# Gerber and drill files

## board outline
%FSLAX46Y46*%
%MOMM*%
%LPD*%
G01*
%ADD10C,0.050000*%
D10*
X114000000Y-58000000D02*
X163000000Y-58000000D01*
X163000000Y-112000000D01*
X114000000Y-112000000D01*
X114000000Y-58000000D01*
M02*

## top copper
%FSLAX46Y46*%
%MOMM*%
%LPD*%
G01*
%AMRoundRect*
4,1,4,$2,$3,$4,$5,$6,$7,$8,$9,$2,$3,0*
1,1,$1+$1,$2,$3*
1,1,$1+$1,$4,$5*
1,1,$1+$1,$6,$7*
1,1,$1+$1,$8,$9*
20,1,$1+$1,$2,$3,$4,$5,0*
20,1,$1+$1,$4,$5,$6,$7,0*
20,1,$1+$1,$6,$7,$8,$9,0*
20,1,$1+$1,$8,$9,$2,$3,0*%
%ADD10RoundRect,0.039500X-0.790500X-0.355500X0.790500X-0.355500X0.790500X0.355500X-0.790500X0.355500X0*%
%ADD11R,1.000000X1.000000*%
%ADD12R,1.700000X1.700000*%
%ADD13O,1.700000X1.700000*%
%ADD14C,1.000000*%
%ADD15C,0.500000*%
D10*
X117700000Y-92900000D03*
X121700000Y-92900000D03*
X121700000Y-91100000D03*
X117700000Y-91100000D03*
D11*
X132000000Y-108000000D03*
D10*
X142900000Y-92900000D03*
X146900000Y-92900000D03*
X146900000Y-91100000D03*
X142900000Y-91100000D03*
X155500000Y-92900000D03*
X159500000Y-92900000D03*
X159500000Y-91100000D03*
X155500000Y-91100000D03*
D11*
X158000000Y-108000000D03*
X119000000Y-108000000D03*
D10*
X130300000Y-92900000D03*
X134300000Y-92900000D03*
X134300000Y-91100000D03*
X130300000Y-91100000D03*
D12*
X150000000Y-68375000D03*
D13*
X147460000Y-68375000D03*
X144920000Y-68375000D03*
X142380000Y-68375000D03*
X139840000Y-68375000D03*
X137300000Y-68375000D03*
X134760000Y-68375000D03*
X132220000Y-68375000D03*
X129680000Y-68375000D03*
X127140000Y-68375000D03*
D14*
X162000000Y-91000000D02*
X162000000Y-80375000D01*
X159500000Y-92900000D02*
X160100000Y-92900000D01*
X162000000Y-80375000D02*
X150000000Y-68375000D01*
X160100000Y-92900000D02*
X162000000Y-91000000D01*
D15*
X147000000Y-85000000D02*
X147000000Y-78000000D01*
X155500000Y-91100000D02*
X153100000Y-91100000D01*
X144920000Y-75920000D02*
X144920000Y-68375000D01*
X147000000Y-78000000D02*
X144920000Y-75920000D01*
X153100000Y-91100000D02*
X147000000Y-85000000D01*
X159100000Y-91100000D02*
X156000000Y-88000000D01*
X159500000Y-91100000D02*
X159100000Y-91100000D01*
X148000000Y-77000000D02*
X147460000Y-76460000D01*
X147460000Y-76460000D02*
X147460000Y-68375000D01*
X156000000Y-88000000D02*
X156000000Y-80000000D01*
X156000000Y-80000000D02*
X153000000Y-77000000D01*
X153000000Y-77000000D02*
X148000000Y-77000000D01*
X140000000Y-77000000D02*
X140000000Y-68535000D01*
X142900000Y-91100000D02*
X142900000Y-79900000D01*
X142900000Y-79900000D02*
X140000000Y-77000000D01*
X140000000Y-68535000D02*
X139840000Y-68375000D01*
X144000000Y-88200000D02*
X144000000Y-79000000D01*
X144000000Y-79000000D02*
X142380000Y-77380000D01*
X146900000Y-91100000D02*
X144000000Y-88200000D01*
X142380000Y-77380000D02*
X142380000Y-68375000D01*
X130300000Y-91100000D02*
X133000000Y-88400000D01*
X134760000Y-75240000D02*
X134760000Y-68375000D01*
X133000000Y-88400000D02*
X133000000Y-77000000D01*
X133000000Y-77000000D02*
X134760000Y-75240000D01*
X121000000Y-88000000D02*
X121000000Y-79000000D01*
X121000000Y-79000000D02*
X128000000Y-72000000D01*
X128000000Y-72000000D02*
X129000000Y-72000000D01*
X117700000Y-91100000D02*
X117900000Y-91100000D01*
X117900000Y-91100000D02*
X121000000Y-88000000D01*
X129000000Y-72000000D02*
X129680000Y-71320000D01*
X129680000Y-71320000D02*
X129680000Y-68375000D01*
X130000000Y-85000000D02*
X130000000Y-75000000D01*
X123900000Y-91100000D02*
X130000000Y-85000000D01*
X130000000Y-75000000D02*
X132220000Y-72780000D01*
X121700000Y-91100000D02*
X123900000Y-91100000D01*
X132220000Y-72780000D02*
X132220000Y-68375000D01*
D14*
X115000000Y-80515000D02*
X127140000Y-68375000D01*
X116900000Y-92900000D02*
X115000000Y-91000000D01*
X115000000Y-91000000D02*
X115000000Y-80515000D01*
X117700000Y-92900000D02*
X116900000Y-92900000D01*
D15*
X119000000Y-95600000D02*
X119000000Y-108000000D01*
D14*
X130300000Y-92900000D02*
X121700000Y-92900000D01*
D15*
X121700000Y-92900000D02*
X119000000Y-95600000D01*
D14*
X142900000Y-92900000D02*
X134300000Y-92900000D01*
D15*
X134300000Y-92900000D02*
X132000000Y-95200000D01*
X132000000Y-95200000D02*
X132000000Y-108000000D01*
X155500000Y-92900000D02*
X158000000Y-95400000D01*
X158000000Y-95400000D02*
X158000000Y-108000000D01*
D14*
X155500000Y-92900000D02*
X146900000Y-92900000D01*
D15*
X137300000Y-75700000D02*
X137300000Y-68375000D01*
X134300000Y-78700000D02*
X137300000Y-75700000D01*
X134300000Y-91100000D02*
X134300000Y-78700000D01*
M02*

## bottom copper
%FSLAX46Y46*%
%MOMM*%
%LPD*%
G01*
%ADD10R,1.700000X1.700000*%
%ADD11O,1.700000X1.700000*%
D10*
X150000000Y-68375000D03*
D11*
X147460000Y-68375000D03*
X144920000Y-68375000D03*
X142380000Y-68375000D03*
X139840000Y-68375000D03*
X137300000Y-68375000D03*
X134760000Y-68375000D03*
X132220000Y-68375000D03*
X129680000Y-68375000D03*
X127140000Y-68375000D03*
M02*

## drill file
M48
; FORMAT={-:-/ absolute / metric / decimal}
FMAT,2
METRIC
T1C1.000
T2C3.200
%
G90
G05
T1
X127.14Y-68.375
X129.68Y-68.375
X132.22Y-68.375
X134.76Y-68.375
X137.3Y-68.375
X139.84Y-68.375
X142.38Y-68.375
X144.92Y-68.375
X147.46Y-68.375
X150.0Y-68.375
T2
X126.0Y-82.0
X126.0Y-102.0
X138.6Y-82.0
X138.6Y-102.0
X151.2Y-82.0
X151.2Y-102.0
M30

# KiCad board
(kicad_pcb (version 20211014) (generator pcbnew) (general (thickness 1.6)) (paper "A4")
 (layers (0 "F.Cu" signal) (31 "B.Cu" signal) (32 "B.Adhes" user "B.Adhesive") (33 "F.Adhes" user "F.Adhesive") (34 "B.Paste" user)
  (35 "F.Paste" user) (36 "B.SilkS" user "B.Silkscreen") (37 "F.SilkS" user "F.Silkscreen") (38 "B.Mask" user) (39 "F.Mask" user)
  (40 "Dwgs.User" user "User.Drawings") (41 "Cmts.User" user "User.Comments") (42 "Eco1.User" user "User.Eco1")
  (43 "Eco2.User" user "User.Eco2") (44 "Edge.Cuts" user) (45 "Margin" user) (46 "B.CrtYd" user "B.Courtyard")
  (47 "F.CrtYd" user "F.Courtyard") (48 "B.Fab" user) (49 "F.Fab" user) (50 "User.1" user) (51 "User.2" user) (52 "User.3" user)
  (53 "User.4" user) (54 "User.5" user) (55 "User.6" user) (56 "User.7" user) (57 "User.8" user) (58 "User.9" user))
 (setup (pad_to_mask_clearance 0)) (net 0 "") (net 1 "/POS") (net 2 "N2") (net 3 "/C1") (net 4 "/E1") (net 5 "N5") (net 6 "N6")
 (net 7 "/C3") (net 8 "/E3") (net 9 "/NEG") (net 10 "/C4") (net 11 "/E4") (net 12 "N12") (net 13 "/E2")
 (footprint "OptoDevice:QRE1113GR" (layer "F.Cu") (at 119.7 92)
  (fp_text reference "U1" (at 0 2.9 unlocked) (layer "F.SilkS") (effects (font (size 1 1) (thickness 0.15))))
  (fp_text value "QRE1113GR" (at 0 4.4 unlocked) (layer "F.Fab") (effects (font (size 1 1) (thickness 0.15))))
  (pad "1" smd roundrect (at -2 0.9) (size 1.66 0.79) (layers "F.Cu" "F.Paste" "F.Mask") (roundrect_rratio 0.05) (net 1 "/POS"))
  (pad "2" smd roundrect (at 2 0.9) (size 1.66 0.79) (layers "F.Cu" "F.Paste" "F.Mask") (roundrect_rratio 0.05) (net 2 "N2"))
  (pad "3" smd roundrect (at 2 -0.9) (size 1.66 0.79) (layers "F.Cu" "F.Paste" "F.Mask") (roundrect_rratio 0.05) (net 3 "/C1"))
  (pad "4" smd roundrect (at -2 -0.9) (size 1.66 0.79) (layers "F.Cu" "F.Paste" "F.Mask") (roundrect_rratio 0.05) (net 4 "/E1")))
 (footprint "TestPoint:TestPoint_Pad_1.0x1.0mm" (layer "F.Cu") (at 132 108)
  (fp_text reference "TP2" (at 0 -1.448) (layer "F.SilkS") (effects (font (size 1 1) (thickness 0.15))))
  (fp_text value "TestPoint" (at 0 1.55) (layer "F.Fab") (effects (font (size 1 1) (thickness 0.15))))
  (pad "1" smd rect locked (at 0 0) (size 1 1) (layers "F.Cu" "F.Mask") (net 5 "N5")))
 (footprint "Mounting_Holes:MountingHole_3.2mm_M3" (layer "F.Cu") (at 126 102)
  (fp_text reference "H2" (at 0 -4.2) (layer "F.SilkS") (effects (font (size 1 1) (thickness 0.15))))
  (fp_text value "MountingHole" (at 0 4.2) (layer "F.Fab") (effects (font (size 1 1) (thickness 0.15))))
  (pad "" np_thru_hole circle (at 0 0) (size 3.2 3.2) (drill 3.2) (layers *.Cu *.Mask)))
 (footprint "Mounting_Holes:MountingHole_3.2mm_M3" (layer "F.Cu") (at 151.2 102)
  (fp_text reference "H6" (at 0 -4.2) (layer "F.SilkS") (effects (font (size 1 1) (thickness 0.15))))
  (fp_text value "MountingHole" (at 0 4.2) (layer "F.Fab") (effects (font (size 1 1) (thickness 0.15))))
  (pad "" np_thru_hole circle (at 0 0) (size 3.2 3.2) (drill 3.2) (layers *.Cu *.Mask)))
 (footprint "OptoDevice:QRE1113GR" (layer "F.Cu") (at 144.9 92)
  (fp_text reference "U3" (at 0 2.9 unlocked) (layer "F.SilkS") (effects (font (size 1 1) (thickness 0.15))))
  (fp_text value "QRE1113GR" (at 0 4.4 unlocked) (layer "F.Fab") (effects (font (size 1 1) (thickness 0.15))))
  (pad "1" smd roundrect (at -2 0.9) (size 1.66 0.79) (layers "F.Cu" "F.Paste" "F.Mask") (roundrect_rratio 0.05) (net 5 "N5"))
  (pad "2" smd roundrect (at 2 0.9) (size 1.66 0.79) (layers "F.Cu" "F.Paste" "F.Mask") (roundrect_rratio 0.05) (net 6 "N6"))
  (pad "3" smd roundrect (at 2 -0.9) (size 1.66 0.79) (layers "F.Cu" "F.Paste" "F.Mask") (roundrect_rratio 0.05) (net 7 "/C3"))
  (pad "4" smd roundrect (at -2 -0.9) (size 1.66 0.79) (layers "F.Cu" "F.Paste" "F.Mask") (roundrect_rratio 0.05) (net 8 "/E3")))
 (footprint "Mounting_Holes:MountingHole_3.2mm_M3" (layer "F.Cu") (at 138.6 102)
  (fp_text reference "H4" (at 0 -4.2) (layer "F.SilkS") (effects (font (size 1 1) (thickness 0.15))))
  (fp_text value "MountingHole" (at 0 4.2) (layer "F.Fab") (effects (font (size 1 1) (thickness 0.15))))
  (pad "" np_thru_hole circle (at 0 0) (size 3.2 3.2) (drill 3.2) (layers *.Cu *.Mask)))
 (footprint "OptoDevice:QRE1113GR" (layer "F.Cu") (at 157.5 92)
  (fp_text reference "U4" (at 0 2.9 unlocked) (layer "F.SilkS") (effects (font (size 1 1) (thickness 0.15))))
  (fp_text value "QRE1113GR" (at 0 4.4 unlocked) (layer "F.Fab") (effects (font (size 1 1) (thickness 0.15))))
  (pad "1" smd roundrect (at -2 0.9) (size 1.66 0.79) (layers "F.Cu" "F.Paste" "F.Mask") (roundrect_rratio 0.05) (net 6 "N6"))
  (pad "2" smd roundrect (at 2 0.9) (size 1.66 0.79) (layers "F.Cu" "F.Paste" "F.Mask") (roundrect_rratio 0.05) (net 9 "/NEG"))
  (pad "3" smd roundrect (at 2 -0.9) (size 1.66 0.79) (layers "F.Cu" "F.Paste" "F.Mask") (roundrect_rratio 0.05) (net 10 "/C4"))
  (pad "4" smd roundrect (at -2 -0.9) (size 1.66 0.79) (layers "F.Cu" "F.Paste" "F.Mask") (roundrect_rratio 0.05) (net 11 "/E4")))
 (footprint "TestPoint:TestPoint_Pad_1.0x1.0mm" (layer "F.Cu") (at 158 108)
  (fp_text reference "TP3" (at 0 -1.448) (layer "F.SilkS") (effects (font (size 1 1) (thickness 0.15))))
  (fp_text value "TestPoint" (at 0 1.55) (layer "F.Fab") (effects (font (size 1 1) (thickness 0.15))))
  (pad "1" smd rect locked (at 0 0) (size 1 1) (layers "F.Cu" "F.Mask") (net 6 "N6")))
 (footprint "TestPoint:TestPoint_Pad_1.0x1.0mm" (layer "F.Cu") (at 119 108)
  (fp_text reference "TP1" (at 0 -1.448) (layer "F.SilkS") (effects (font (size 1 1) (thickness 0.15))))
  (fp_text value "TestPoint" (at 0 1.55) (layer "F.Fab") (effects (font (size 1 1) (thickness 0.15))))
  (pad "1" smd rect locked (at 0 0) (size 1 1) (layers "F.Cu" "F.Mask") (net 2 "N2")))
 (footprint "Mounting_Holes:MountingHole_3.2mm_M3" (layer "F.Cu") (at 138.6 82)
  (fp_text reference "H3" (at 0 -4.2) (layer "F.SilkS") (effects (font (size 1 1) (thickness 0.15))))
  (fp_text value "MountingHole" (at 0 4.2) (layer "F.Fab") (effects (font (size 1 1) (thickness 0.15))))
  (pad "" np_thru_hole circle (at 0 0) (size 3.2 3.2) (drill 3.2) (layers *.Cu *.Mask)))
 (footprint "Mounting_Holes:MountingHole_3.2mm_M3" (layer "F.Cu") (at 151.2 82)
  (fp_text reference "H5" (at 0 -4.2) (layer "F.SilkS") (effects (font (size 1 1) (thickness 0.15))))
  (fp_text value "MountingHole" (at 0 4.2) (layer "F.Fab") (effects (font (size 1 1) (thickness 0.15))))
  (pad "" np_thru_hole circle (at 0 0) (size 3.2 3.2) (drill 3.2) (layers *.Cu *.Mask)))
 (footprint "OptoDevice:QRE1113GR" (layer "F.Cu") (at 132.3 92)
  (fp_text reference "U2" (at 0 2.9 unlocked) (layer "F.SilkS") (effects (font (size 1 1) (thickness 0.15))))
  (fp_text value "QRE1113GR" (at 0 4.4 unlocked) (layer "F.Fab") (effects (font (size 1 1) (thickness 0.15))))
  (pad "1" smd roundrect (at -2 0.9) (size 1.66 0.79) (layers "F.Cu" "F.Paste" "F.Mask") (roundrect_rratio 0.05) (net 2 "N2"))
  (pad "2" smd roundrect (at 2 0.9) (size 1.66 0.79) (layers "F.Cu" "F.Paste" "F.Mask") (roundrect_rratio 0.05) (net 5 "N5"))
  (pad "3" smd roundrect (at 2 -0.9) (size 1.66 0.79) (layers "F.Cu" "F.Paste" "F.Mask") (roundrect_rratio 0.05) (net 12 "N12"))
  (pad "4" smd roundrect (at -2 -0.9) (size 1.66 0.79) (layers "F.Cu" "F.Paste" "F.Mask") (roundrect_rratio 0.05) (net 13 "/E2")))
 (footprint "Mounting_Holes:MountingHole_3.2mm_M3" (layer "F.Cu") (at 126 82)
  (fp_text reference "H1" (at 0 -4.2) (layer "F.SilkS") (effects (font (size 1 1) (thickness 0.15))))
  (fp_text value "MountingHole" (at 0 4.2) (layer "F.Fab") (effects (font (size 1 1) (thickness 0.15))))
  (pad "" np_thru_hole circle (at 0 0) (size 3.2 3.2) (drill 3.2) (layers *.Cu *.Mask)))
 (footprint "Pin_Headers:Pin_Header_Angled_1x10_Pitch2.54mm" (layer "B.Cu") (at 150 68.375 90)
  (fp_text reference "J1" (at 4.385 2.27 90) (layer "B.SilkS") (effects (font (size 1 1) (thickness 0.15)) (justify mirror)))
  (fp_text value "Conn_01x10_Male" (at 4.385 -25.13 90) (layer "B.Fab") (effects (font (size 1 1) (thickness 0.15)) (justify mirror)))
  (pad "1" thru_hole rect locked (at 0 0 90) (size 1.7 1.7) (drill 1) (layers *.Cu *.Mask) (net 9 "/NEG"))
  (pad "2" thru_hole oval locked (at 0 -2.54 90) (size 1.7 1.7) (drill 1) (layers *.Cu *.Mask) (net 10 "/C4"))
  (pad "3" thru_hole oval locked (at 0 -5.08 90) (size 1.7 1.7) (drill 1) (layers *.Cu *.Mask) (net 11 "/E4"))
  (pad "4" thru_hole oval locked (at 0 -7.62 90) (size 1.7 1.7) (drill 1) (layers *.Cu *.Mask) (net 7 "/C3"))
  (pad "5" thru_hole oval locked (at 0 -10.16 90) (size 1.7 1.7) (drill 1) (layers *.Cu *.Mask) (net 8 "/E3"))
  (pad "6" thru_hole oval locked (at 0 -12.7 90) (size 1.7 1.7) (drill 1) (layers *.Cu *.Mask) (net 12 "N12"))
  (pad "7" thru_hole oval locked (at 0 -15.24 90) (size 1.7 1.7) (drill 1) (layers *.Cu *.Mask) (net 13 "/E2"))
  (pad "8" thru_hole oval locked (at 0 -17.78 90) (size 1.7 1.7) (drill 1) (layers *.Cu *.Mask) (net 3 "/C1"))
  (pad "9" thru_hole oval locked (at 0 -20.32 90) (size 1.7 1.7) (drill 1) (layers *.Cu *.Mask) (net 4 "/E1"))
  (pad "10" thru_hole oval locked (at 0 -22.86 90) (size 1.7 1.7) (drill 1) (layers *.Cu *.Mask) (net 1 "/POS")))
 (gr_rect (start 114 58) (end 163 112) (layer "Edge.Cuts") (width 0.05) (fill none))
 (segment (start 162 91) (end 162 80.375) (width 1) (layer "F.Cu") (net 9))
 (segment (start 159.5 92.9) (end 160.1 92.9) (width 1) (layer "F.Cu") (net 9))
 (segment (start 162 80.375) (end 150 68.375) (width 1) (layer "F.Cu") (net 9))
 (segment (start 160.1 92.9) (end 162 91) (width 1) (layer "F.Cu") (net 9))
 (segment (start 147 85) (end 147 78) (width 0.5) (layer "F.Cu") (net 11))
 (segment (start 155.5 91.1) (end 153.1 91.1) (width 0.5) (layer "F.Cu") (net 11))
 (segment (start 144.92 75.92) (end 144.92 68.375) (width 0.5) (layer "F.Cu") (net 11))
 (segment (start 147 78) (end 144.92 75.92) (width 0.5) (layer "F.Cu") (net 11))
 (segment (start 153.1 91.1) (end 147 85) (width 0.5) (layer "F.Cu") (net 11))
 (segment (start 159.1 91.1) (end 156 88) (width 0.5) (layer "F.Cu") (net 10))
 (segment (start 159.5 91.1) (end 159.1 91.1) (width 0.5) (layer "F.Cu") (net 10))
 (segment (start 148 77) (end 147.46 76.46) (width 0.5) (layer "F.Cu") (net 10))
 (segment (start 147.46 76.46) (end 147.46 68.375) (width 0.5) (layer "F.Cu") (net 10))
 (segment (start 156 88) (end 156 80) (width 0.5) (layer "F.Cu") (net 10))
 (segment (start 156 80) (end 153 77) (width 0.5) (layer "F.Cu") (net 10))
 (segment (start 153 77) (end 148 77) (width 0.5) (layer "F.Cu") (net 10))
 (segment (start 140 77) (end 140 68.535) (width 0.5) (layer "F.Cu") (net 8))
 (segment (start 142.9 91.1) (end 142.9 79.9) (width 0.5) (layer "F.Cu") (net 8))
 (segment (start 142.9 79.9) (end 140 77) (width 0.5) (layer "F.Cu") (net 8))
 (segment (start 140 68.535) (end 139.84 68.375) (width 0.5) (layer "F.Cu") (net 8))
 (segment (start 144 88.2) (end 144 79) (width 0.5) (layer "F.Cu") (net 7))
 (segment (start 144 79) (end 142.38 77.38) (width 0.5) (layer "F.Cu") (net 7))
 (segment (start 146.9 91.1) (end 144 88.2) (width 0.5) (layer "F.Cu") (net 7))
 (segment (start 142.38 77.38) (end 142.38 68.375) (width 0.5) (layer "F.Cu") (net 7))
 (segment (start 130.3 91.1) (end 133 88.4) (width 0.5) (layer "F.Cu") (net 13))
 (segment (start 134.76 75.24) (end 134.76 68.375) (width 0.5) (layer "F.Cu") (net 13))
 (segment (start 133 88.4) (end 133 77) (width 0.5) (layer "F.Cu") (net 13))
 (segment (start 133 77) (end 134.76 75.24) (width 0.5) (layer "F.Cu") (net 13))
 (segment (start 121 88) (end 121 79) (width 0.5) (layer "F.Cu") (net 4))
 (segment (start 121 79) (end 128 72) (width 0.5) (layer "F.Cu") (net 4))
 (segment (start 128 72) (end 129 72) (width 0.5) (layer "F.Cu") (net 4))
 (segment (start 117.7 91.1) (end 117.9 91.1) (width 0.5) (layer "F.Cu") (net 4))
 (segment (start 117.9 91.1) (end 121 88) (width 0.5) (layer "F.Cu") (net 4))
 (segment (start 129 72) (end 129.68 71.32) (width 0.5) (layer "F.Cu") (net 4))
 (segment (start 129.68 71.32) (end 129.68 68.375) (width 0.5) (layer "F.Cu") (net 4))
 (segment (start 130 85) (end 130 75) (width 0.5) (layer "F.Cu") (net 3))
 (segment (start 123.9 91.1) (end 130 85) (width 0.5) (layer "F.Cu") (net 3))
 (segment (start 130 75) (end 132.22 72.78) (width 0.5) (layer "F.Cu") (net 3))
 (segment (start 121.7 91.1) (end 123.9 91.1) (width 0.5) (layer "F.Cu") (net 3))
 (segment (start 132.22 72.78) (end 132.22 68.375) (width 0.5) (layer "F.Cu") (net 3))
 (segment (start 115 80.515) (end 127.14 68.375) (width 1) (layer "F.Cu") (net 1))
 (segment (start 116.9 92.9) (end 115 91) (width 1) (layer "F.Cu") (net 1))
 (segment (start 115 91) (end 115 80.515) (width 1) (layer "F.Cu") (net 1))
 (segment (start 117.7 92.9) (end 116.9 92.9) (width 1) (layer "F.Cu") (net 1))
 (segment (start 119 95.6) (end 119 108) (width 0.5) (layer "F.Cu") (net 2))
 (segment (start 130.3 92.9) (end 121.7 92.9) (width 1) (layer "F.Cu") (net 2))
 (segment (start 121.7 92.9) (end 119 95.6) (width 0.5) (layer "F.Cu") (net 2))
 (segment (start 142.9 92.9) (end 134.3 92.9) (width 1) (layer "F.Cu") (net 5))
 (segment (start 134.3 92.9) (end 132 95.2) (width 0.5) (layer "F.Cu") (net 5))
 (segment (start 132 95.2) (end 132 108) (width 0.5) (layer "F.Cu") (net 5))
 (segment (start 155.5 92.9) (end 158 95.4) (width 0.5) (layer "F.Cu") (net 6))
 (segment (start 158 95.4) (end 158 108) (width 0.5) (layer "F.Cu") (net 6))
 (segment (start 155.5 92.9) (end 146.9 92.9) (width 1) (layer "F.Cu") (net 6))
 (segment (start 137.3 75.7) (end 137.3 68.375) (width 0.5) (layer "F.Cu") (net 12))
 (segment (start 134.3 78.7) (end 137.3 75.7) (width 0.5) (layer "F.Cu") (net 12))
 (segment (start 134.3 91.1) (end 134.3 78.7) (width 0.5) (layer "F.Cu") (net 12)))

